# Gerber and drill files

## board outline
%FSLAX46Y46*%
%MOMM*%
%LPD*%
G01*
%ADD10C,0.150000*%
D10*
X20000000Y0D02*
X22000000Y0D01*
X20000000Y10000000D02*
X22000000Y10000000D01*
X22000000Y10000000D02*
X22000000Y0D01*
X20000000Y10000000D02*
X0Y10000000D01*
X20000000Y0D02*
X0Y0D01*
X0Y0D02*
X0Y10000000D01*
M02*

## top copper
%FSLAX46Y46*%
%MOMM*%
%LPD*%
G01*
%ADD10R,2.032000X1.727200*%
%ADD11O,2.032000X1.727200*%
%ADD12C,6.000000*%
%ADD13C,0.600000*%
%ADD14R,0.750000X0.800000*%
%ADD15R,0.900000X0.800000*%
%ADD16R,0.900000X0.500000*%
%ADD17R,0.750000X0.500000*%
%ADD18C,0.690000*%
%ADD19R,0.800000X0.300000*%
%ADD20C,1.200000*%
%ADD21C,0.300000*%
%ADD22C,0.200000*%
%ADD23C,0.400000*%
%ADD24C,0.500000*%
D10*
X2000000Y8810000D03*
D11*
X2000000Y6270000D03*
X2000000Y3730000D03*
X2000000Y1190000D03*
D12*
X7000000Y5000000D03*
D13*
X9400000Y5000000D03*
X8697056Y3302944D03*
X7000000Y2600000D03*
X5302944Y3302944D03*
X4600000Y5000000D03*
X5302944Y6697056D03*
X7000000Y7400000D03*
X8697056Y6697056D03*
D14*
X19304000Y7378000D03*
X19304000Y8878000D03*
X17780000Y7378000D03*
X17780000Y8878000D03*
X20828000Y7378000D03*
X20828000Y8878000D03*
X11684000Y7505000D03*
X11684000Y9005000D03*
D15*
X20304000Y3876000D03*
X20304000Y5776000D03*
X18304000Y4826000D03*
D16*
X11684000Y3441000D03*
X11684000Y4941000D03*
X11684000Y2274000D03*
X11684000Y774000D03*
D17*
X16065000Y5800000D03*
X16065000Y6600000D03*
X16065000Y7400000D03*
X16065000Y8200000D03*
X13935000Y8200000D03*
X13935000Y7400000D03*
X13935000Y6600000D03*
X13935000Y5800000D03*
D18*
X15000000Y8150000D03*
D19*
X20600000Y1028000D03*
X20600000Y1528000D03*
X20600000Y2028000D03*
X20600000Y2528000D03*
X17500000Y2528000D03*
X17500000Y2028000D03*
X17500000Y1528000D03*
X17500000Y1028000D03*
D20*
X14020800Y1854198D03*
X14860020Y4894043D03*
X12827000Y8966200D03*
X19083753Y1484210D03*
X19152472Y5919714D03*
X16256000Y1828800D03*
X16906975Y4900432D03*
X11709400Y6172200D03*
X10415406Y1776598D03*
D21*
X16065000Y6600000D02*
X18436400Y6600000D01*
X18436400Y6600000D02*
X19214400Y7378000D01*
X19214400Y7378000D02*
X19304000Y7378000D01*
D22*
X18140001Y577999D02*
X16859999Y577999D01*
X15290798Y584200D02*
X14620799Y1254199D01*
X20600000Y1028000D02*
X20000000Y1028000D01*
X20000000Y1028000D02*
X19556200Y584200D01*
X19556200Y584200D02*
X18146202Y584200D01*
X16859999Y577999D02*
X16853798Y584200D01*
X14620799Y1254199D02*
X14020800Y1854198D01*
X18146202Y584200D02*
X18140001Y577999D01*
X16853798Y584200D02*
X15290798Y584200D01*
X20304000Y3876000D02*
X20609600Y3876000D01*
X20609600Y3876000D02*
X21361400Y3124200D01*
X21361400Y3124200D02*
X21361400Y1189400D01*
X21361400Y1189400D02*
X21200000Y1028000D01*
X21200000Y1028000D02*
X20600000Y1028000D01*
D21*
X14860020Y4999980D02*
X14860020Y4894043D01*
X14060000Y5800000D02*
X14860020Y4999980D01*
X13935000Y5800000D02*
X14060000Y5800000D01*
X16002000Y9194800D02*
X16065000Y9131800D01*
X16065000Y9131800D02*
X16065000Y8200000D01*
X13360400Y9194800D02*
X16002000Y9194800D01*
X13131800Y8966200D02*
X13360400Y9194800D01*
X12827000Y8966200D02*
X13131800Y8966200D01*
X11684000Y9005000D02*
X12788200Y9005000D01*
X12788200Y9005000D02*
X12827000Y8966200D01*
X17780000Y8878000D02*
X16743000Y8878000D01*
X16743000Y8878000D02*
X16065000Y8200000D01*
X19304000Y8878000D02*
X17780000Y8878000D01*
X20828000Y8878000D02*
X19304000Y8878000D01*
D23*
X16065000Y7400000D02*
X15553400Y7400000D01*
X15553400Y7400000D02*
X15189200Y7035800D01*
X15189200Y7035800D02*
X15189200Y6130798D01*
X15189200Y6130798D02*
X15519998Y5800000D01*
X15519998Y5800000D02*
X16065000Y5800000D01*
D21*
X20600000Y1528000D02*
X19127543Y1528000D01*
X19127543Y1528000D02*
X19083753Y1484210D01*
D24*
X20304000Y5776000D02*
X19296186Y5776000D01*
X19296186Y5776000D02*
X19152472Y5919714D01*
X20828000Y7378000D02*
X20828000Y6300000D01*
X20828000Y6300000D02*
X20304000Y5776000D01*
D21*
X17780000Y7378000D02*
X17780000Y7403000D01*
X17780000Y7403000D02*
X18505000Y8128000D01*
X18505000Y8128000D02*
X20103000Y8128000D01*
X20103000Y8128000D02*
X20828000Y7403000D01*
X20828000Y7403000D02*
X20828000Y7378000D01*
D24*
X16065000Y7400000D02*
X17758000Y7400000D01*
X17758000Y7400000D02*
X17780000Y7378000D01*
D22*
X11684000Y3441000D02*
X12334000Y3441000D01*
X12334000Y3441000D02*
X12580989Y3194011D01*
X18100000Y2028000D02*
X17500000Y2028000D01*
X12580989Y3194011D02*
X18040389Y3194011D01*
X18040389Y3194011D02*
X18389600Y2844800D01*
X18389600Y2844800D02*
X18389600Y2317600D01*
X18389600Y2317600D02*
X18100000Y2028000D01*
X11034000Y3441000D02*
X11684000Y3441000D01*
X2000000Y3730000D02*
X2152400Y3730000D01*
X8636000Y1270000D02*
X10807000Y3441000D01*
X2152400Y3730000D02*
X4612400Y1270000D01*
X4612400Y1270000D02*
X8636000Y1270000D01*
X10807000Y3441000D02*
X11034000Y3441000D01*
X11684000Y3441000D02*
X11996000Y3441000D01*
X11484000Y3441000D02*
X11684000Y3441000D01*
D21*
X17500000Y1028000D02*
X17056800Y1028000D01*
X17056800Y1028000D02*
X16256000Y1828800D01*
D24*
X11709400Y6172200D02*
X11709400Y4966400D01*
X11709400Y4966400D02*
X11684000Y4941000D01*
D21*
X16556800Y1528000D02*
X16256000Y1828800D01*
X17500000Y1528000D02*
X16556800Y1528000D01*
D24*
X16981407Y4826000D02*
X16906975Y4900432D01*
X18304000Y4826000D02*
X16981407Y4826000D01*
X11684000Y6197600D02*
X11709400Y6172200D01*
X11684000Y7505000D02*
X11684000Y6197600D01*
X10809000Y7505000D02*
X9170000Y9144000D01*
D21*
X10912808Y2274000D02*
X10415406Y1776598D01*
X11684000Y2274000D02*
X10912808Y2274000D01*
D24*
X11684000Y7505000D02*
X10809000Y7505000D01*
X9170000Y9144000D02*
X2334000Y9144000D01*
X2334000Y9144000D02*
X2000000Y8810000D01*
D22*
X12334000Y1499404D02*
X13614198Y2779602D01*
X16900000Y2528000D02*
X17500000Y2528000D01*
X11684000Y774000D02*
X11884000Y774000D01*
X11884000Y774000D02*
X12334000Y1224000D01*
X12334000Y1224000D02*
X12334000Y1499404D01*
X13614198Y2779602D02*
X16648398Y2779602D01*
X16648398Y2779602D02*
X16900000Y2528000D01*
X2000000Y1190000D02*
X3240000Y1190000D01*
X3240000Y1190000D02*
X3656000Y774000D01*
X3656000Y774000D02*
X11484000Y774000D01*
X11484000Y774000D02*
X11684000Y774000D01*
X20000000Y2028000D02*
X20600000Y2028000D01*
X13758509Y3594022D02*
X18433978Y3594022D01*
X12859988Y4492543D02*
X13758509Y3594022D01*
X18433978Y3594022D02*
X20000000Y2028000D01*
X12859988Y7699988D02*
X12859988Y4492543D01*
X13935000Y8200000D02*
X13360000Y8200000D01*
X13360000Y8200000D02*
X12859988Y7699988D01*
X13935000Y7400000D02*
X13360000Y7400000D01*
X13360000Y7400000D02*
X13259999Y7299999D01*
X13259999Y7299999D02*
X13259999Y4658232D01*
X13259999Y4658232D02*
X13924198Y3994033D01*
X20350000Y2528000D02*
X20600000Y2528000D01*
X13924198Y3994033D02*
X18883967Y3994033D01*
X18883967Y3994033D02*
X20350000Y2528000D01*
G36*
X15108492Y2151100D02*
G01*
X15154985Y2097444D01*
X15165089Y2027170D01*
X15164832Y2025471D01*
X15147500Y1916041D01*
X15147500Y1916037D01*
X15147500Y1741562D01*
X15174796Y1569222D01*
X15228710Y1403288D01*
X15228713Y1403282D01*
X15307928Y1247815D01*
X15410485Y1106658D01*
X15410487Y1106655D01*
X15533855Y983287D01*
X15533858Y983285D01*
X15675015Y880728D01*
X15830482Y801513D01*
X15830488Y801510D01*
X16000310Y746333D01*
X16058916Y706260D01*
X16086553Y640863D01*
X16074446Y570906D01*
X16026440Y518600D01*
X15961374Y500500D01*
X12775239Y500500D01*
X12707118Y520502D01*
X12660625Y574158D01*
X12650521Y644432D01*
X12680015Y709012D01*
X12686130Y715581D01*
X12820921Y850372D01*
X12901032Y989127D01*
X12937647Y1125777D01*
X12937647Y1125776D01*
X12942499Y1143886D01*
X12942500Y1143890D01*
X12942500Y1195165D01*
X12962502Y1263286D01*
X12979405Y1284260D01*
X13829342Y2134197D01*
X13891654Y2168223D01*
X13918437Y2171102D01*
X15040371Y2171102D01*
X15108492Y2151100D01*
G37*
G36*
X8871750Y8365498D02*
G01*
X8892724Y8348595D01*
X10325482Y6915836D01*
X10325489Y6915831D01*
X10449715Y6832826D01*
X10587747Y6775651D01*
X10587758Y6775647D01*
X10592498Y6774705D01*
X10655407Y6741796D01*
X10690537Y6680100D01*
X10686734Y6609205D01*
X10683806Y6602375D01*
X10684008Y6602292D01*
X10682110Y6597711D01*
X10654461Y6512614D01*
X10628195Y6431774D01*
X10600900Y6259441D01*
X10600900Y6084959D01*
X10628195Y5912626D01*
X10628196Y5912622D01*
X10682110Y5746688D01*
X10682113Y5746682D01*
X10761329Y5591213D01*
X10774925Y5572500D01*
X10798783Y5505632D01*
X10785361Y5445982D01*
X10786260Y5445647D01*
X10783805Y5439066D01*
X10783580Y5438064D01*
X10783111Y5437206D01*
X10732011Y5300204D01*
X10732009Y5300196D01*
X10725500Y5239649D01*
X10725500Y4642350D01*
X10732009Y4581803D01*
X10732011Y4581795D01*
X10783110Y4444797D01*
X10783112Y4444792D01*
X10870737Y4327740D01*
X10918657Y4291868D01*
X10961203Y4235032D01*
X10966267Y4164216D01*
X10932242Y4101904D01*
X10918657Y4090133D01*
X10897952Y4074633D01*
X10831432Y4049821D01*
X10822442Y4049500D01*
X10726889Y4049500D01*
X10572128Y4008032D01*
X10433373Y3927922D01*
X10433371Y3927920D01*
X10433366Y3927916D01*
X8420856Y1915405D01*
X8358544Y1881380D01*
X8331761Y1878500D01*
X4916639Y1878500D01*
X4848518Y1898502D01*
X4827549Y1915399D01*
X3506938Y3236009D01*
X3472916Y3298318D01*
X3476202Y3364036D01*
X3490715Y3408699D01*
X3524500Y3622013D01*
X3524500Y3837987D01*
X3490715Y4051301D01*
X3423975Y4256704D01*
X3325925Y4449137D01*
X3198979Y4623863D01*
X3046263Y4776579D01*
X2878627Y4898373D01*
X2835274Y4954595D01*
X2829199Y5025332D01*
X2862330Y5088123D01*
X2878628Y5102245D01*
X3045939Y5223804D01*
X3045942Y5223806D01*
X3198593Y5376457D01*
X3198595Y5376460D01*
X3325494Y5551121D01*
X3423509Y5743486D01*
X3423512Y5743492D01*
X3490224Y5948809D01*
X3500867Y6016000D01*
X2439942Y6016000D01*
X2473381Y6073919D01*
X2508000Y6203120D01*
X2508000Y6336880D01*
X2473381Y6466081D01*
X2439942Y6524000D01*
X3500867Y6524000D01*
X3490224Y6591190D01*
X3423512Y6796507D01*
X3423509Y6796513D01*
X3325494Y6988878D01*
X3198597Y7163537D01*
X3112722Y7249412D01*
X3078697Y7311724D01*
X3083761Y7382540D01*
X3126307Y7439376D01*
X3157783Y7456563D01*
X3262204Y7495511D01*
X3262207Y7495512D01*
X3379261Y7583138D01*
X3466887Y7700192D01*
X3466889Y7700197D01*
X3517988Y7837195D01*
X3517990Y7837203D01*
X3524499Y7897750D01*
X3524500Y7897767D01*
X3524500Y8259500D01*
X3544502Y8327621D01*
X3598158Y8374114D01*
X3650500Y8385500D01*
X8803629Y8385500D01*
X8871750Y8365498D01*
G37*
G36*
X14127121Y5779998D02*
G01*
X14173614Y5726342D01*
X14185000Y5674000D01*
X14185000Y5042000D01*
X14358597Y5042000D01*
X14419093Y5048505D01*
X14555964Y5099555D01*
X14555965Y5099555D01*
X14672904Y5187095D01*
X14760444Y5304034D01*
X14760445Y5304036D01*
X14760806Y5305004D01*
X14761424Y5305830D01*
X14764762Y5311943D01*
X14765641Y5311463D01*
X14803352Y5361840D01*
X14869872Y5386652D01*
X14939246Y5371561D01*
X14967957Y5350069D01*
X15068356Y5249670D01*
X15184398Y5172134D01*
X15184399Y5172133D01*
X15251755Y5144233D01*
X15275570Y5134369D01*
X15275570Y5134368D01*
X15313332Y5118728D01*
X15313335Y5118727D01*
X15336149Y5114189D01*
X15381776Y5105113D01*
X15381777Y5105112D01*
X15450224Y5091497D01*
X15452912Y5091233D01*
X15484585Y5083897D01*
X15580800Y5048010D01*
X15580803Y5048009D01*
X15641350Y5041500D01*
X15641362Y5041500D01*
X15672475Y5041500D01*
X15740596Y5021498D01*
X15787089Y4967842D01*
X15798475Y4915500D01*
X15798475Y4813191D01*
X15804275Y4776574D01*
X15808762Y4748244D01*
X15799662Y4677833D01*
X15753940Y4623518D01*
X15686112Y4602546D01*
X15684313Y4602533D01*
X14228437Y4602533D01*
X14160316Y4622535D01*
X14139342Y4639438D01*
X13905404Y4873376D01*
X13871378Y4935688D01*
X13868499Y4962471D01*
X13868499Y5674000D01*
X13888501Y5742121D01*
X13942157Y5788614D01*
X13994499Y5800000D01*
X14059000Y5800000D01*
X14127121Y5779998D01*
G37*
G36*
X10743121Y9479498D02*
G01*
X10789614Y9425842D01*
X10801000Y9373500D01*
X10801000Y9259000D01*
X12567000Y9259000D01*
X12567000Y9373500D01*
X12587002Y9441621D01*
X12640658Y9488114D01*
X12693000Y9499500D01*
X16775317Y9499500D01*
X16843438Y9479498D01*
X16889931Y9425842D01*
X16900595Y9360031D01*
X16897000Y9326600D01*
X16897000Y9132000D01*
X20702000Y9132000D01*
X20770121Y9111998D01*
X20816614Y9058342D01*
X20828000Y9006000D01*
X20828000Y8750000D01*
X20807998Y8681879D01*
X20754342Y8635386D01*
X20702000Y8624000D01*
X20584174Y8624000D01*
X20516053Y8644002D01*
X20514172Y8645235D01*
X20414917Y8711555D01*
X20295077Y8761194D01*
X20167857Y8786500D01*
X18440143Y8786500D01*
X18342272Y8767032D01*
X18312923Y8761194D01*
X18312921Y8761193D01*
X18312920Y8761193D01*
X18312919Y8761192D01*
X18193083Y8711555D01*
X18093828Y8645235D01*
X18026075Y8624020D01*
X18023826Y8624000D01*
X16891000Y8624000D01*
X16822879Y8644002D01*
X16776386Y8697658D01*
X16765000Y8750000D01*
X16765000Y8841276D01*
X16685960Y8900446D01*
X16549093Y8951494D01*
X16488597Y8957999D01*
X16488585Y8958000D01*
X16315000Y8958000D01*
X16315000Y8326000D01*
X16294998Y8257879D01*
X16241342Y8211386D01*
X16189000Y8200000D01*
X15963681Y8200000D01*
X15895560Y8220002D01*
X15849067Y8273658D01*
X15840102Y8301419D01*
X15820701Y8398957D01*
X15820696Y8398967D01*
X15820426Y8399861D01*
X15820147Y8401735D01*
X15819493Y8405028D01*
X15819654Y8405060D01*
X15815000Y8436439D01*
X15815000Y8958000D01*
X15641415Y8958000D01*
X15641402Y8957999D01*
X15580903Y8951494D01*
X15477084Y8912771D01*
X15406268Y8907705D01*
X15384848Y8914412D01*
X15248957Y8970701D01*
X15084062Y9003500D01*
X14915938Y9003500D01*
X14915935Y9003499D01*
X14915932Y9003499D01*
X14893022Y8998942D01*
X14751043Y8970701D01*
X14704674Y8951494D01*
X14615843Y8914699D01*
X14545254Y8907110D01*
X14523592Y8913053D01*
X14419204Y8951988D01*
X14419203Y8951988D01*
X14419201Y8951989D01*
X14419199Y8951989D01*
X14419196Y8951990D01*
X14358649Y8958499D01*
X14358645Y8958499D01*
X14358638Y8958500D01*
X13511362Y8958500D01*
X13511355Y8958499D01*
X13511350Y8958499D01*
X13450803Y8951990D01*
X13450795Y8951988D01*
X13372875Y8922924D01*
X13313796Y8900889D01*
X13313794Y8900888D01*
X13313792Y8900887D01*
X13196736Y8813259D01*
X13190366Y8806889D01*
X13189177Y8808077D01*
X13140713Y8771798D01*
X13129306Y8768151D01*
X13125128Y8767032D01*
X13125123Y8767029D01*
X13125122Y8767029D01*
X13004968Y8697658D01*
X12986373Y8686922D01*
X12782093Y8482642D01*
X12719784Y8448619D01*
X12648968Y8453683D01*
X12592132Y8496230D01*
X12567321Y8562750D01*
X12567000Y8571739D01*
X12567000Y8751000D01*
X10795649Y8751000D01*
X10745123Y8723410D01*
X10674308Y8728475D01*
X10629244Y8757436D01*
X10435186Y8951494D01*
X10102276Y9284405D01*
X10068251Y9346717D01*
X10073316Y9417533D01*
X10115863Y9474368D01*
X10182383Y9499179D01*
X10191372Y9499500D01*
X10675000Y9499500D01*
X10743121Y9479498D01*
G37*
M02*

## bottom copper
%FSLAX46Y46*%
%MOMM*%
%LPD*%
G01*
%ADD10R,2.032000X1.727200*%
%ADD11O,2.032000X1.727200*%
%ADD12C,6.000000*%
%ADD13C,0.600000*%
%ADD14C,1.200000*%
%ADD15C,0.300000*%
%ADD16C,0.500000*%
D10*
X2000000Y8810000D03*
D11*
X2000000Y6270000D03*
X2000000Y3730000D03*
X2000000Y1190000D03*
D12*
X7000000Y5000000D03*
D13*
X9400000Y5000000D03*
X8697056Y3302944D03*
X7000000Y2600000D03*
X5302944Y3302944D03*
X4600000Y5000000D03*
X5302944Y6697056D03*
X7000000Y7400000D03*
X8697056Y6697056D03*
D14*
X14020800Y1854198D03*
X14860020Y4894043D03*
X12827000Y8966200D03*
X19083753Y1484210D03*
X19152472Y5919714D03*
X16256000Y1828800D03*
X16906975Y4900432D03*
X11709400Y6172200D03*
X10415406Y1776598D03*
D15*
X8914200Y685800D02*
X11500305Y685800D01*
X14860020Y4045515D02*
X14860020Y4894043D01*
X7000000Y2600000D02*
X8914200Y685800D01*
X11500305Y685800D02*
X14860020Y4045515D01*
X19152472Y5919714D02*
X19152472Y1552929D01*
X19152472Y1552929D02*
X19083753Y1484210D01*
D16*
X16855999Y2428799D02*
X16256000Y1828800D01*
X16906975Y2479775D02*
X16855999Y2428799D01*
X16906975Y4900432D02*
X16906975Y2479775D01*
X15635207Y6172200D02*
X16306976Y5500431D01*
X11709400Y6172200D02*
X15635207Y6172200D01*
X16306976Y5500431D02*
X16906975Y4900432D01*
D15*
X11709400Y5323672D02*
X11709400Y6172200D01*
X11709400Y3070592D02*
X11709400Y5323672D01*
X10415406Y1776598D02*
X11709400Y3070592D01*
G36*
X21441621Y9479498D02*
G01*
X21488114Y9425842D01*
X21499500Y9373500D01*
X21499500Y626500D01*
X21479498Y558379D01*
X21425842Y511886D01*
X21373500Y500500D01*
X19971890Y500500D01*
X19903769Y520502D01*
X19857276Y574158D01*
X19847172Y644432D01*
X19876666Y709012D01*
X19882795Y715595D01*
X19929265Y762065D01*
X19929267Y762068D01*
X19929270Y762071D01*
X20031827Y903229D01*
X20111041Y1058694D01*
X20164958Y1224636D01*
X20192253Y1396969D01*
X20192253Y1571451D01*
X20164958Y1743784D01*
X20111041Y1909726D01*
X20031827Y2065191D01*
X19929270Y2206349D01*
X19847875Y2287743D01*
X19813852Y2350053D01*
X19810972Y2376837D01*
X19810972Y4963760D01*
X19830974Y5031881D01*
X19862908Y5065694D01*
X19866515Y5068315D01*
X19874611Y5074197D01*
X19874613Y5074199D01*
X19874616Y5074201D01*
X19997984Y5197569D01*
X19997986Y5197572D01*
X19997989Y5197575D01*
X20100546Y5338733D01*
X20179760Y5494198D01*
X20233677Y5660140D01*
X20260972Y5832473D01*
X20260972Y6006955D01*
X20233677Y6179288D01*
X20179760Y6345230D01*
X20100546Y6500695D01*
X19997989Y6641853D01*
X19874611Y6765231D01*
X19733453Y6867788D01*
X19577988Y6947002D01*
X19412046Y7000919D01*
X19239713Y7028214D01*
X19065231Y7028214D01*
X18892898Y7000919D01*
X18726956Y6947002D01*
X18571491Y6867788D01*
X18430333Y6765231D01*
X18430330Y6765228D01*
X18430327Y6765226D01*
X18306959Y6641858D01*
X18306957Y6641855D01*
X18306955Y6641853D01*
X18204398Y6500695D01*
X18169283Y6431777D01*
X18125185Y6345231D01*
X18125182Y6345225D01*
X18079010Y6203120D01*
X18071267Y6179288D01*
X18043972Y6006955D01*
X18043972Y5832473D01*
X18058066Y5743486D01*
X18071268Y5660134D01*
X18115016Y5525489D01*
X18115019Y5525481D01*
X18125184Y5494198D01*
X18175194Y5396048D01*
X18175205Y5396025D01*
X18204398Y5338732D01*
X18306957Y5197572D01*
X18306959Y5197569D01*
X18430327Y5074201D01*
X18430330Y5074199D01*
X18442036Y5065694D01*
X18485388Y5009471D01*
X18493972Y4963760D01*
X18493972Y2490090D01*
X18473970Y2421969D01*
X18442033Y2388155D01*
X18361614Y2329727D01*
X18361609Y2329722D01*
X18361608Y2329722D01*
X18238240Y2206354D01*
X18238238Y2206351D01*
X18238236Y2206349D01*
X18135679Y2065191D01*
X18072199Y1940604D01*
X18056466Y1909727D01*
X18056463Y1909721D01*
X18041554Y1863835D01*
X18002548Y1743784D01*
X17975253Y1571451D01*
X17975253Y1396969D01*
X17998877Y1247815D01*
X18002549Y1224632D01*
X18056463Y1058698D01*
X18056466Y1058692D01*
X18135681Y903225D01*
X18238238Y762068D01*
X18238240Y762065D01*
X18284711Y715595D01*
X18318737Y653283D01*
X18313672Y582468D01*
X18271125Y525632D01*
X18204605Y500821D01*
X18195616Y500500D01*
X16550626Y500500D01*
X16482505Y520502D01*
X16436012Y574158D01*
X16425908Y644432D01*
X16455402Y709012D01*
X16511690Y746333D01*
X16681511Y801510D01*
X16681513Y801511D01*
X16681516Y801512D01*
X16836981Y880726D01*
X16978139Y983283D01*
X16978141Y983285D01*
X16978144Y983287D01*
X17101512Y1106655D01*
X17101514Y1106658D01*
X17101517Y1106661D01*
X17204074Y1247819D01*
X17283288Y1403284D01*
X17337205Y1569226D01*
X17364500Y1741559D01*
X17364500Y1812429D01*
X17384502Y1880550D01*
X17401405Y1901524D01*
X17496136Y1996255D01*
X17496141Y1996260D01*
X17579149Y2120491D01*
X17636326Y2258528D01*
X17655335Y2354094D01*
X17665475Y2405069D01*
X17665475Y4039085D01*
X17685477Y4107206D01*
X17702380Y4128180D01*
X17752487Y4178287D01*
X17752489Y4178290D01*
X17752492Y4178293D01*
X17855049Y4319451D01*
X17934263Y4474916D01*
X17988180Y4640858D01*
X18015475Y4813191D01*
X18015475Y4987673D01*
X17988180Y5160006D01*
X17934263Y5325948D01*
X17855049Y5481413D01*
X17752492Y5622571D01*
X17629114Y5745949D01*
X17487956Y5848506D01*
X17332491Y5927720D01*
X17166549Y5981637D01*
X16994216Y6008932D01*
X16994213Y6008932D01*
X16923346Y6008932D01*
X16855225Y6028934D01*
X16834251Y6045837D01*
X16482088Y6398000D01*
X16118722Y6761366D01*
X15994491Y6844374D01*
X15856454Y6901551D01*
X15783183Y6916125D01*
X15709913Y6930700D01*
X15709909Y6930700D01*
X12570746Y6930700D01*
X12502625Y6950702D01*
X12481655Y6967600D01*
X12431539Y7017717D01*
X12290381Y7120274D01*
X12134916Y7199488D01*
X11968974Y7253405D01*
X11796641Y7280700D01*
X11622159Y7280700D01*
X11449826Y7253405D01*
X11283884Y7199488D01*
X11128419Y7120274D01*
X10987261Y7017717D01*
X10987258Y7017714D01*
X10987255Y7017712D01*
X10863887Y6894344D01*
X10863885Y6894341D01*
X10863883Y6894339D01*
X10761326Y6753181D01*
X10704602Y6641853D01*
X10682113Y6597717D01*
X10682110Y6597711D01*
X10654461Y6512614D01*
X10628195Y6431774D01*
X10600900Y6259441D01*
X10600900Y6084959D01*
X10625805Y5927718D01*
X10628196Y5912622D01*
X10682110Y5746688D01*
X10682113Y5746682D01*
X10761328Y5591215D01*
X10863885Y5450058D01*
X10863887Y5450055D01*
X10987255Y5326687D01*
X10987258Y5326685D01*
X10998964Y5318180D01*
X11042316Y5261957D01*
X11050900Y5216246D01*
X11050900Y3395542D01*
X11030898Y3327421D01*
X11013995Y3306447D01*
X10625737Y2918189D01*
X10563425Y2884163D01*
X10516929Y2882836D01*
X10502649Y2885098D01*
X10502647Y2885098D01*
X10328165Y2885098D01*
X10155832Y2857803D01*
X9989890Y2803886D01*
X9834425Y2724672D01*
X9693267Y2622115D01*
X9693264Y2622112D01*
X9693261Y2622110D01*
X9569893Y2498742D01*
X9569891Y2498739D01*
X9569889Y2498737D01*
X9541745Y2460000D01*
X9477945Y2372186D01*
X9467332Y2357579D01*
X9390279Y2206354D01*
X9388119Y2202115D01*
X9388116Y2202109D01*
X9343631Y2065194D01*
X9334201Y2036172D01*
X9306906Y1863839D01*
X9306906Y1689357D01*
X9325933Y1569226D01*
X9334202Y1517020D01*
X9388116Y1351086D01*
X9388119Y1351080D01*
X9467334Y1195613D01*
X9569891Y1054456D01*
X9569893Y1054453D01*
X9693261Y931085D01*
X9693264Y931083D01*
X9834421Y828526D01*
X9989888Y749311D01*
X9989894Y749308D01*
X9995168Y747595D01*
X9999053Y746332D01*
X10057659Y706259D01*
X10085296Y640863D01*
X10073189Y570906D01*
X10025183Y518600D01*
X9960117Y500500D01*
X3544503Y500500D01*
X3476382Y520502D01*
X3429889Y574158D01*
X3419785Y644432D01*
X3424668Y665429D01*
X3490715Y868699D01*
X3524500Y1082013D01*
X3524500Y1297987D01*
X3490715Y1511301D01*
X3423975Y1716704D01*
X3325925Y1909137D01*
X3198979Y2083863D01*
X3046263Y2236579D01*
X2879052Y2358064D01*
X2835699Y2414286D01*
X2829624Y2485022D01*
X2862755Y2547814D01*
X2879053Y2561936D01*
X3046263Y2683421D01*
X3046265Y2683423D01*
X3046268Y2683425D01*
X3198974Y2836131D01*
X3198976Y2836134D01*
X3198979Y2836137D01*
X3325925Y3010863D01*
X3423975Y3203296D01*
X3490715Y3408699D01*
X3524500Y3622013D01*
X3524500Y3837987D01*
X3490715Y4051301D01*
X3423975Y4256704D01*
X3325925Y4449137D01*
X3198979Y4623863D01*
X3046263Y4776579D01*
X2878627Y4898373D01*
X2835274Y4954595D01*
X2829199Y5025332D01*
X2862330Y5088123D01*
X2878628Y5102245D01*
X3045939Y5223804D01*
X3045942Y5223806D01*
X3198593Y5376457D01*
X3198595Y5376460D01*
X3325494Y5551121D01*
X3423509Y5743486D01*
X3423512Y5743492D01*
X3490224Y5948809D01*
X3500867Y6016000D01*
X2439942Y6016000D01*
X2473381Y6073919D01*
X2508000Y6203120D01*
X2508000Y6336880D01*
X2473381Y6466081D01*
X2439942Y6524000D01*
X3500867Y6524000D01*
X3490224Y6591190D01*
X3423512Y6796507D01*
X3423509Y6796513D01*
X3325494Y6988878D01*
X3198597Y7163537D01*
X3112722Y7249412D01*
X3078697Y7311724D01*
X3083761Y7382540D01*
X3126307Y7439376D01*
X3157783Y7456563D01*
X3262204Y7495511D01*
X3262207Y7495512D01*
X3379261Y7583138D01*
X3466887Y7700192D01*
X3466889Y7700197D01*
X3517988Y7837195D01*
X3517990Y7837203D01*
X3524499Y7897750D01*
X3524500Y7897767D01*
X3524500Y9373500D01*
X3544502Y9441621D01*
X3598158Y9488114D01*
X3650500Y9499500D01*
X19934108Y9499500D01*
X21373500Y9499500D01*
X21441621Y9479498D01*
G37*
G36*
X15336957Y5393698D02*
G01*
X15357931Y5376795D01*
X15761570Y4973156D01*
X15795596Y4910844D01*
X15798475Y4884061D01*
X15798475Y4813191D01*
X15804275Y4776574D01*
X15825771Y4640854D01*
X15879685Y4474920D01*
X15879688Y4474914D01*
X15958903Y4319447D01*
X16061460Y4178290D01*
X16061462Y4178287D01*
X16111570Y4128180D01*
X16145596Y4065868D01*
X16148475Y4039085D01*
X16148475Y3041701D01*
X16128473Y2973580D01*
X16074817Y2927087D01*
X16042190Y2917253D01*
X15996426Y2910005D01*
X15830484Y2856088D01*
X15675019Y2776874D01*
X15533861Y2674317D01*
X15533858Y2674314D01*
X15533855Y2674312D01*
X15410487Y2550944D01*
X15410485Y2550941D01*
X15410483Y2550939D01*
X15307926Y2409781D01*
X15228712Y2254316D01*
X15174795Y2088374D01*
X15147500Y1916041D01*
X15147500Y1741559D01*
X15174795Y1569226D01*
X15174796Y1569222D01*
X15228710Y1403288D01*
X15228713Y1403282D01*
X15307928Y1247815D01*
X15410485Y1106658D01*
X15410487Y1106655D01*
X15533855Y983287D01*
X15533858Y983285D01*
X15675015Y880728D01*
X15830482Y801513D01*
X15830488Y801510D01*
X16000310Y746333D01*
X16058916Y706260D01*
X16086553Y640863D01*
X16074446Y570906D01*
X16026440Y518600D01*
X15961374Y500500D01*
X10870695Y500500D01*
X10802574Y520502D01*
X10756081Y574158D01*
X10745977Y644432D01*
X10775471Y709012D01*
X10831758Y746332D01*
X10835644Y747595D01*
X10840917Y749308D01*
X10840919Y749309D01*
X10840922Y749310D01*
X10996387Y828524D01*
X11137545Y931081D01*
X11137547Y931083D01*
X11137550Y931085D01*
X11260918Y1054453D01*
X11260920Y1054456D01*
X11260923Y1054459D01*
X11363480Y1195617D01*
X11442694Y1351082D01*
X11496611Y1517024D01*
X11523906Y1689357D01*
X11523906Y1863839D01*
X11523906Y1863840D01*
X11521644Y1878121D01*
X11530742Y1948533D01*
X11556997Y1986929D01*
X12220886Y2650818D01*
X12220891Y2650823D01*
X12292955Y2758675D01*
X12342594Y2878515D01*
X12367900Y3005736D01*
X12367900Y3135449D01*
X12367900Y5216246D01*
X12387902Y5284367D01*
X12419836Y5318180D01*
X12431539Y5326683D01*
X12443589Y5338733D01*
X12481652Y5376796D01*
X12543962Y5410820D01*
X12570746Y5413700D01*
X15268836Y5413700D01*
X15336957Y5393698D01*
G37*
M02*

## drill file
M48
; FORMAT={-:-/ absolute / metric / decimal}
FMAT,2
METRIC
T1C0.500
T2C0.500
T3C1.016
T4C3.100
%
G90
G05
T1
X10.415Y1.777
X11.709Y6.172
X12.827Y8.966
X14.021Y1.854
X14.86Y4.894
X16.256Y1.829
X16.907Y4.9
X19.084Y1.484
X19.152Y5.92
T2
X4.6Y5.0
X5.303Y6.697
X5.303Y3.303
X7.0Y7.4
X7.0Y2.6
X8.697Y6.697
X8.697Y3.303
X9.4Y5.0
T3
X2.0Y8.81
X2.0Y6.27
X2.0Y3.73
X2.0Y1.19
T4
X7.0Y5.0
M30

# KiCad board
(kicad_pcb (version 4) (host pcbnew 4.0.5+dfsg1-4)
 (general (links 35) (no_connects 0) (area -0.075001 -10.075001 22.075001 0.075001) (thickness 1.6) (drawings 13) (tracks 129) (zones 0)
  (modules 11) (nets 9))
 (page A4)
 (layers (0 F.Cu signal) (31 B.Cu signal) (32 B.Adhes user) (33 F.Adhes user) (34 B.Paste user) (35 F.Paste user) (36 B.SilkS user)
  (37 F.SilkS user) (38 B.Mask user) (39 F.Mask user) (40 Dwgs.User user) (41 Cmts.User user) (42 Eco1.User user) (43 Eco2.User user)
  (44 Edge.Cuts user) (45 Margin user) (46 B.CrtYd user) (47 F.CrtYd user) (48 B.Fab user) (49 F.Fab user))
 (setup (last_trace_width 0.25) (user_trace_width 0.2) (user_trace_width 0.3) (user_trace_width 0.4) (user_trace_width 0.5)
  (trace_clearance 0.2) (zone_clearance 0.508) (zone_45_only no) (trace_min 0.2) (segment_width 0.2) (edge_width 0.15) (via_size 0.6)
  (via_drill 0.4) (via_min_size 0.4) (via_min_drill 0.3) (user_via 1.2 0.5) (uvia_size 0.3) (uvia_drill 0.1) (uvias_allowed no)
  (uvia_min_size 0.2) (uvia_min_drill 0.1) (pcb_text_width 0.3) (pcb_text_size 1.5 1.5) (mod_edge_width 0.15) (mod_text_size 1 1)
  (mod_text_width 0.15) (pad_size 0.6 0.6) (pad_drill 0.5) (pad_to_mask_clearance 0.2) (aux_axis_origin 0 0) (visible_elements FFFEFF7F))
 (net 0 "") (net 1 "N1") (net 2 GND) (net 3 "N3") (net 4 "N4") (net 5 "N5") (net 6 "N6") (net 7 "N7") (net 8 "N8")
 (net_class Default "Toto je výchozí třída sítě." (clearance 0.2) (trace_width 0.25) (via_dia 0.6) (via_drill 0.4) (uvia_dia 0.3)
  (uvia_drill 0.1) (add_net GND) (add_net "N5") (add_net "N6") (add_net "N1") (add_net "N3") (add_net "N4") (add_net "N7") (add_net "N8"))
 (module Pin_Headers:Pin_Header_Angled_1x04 (layer B.Cu) (at 2 -8.81 180)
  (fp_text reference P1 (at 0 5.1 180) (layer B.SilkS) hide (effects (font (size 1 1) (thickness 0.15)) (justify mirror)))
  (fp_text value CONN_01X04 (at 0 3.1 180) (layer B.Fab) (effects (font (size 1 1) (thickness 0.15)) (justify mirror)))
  (pad 1 thru_hole rect (at 0 0 180) (size 2.032 1.7272) (drill 1.016) (layers *.Cu *.Mask) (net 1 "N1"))
  (pad 2 thru_hole oval (at 0 -2.54 180) (size 2.032 1.7272) (drill 1.016) (layers *.Cu *.Mask) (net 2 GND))
  (pad 3 thru_hole oval (at 0 -5.08 180) (size 2.032 1.7272) (drill 1.016) (layers *.Cu *.Mask) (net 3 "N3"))
  (pad 4 thru_hole oval (at 0 -7.62 180) (size 2.032 1.7272) (drill 1.016) (layers *.Cu *.Mask) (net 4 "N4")))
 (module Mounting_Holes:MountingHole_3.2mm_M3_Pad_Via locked (layer F.Cu) (at 7 -5)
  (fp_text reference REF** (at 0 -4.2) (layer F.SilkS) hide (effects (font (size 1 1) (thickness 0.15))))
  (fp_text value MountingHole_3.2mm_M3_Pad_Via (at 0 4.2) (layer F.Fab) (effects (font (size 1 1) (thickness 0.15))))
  (pad 1 thru_hole circle (at 0 0) (size 6 6) (drill 3.1) (layers *.Cu *.Mask) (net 2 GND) (zone_connect 2))
  (pad "" thru_hole circle (at 2.4 0) (size 0.6 0.6) (drill 0.5) (layers *.Cu *.Mask) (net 2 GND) (zone_connect 2))
  (pad "" thru_hole circle (at 1.697056 1.697056) (size 0.6 0.6) (drill 0.5) (layers *.Cu *.Mask) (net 2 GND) (zone_connect 2))
  (pad "" thru_hole circle (at 0 2.4) (size 0.6 0.6) (drill 0.5) (layers *.Cu *.Mask) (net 2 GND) (zone_connect 2))
  (pad "" thru_hole circle (at -1.697056 1.697056) (size 0.6 0.6) (drill 0.5) (layers *.Cu *.Mask) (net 2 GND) (zone_connect 2))
  (pad "" thru_hole circle (at -2.4 0) (size 0.6 0.6) (drill 0.5) (layers *.Cu *.Mask) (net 2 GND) (zone_connect 2))
  (pad "" thru_hole circle (at -1.697056 -1.697056) (size 0.6 0.6) (drill 0.5) (layers *.Cu *.Mask) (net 2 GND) (zone_connect 2))
  (pad "" thru_hole circle (at 0 -2.4) (size 0.6 0.6) (drill 0.5) (layers *.Cu *.Mask) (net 2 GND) (zone_connect 2))
  (pad "" thru_hole circle (at 1.697056 -1.697056) (size 0.6 0.6) (drill 0.5) (layers *.Cu *.Mask) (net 2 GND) (zone_connect 2)))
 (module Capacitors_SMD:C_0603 (layer F.Cu) (at 19.304 -8.128 90)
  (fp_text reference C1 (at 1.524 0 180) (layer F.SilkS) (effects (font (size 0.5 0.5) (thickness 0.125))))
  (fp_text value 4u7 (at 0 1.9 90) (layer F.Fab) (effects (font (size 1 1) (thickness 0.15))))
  (pad 1 smd rect (at -0.75 0 90) (size 0.8 0.75) (layers F.Cu F.Paste F.Mask) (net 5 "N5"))
  (pad 2 smd rect (at 0.75 0 90) (size 0.8 0.75) (layers F.Cu F.Paste F.Mask) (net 2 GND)))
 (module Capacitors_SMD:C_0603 (layer F.Cu) (at 17.78 -8.128 90)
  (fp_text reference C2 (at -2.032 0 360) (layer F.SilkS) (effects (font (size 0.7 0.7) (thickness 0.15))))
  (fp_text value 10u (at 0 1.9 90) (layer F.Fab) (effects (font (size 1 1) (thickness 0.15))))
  (pad 1 smd rect (at -0.75 0 90) (size 0.8 0.75) (layers F.Cu F.Paste F.Mask) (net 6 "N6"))
  (pad 2 smd rect (at 0.75 0 90) (size 0.8 0.75) (layers F.Cu F.Paste F.Mask) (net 2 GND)))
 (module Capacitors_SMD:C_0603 (layer F.Cu) (at 20.828 -8.128 90)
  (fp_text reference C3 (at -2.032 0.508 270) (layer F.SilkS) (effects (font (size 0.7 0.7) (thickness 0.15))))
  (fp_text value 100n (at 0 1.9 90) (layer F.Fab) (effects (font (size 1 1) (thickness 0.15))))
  (pad 1 smd rect (at -0.75 0 90) (size 0.8 0.75) (layers F.Cu F.Paste F.Mask) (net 6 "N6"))
  (pad 2 smd rect (at 0.75 0 90) (size 0.8 0.75) (layers F.Cu F.Paste F.Mask) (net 2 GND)))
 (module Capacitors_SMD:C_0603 (layer F.Cu) (at 11.684 -8.255 90)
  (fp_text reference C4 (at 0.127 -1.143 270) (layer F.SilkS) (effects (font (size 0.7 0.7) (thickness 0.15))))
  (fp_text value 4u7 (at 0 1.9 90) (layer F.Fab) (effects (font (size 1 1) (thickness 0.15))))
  (pad 1 smd rect (at -0.75 0 90) (size 0.8 0.75) (layers F.Cu F.Paste F.Mask) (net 1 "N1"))
  (pad 2 smd rect (at 0.75 0 90) (size 0.8 0.75) (layers F.Cu F.Paste F.Mask) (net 2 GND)))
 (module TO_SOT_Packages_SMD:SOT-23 (layer F.Cu) (at 19.304 -4.826 180)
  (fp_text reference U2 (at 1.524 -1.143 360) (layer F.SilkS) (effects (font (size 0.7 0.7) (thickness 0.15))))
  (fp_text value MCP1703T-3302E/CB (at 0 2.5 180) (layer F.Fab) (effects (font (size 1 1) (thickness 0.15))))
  (pad 1 smd rect (at -1 -0.95 180) (size 0.9 0.8) (layers F.Cu F.Paste F.Mask) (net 2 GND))
  (pad 2 smd rect (at -1 0.95 180) (size 0.9 0.8) (layers F.Cu F.Paste F.Mask) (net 6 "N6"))
  (pad 3 smd rect (at 1 0 180) (size 0.9 0.8) (layers F.Cu F.Paste F.Mask) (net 1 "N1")))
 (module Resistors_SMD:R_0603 (layer F.Cu) (at 11.684 -4.191 90)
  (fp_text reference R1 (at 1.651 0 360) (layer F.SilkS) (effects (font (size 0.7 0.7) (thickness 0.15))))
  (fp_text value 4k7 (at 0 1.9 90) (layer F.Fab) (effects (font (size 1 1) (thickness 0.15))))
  (pad 1 smd rect (at -0.75 0 90) (size 0.5 0.9) (layers F.Cu F.Paste F.Mask) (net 3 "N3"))
  (pad 2 smd rect (at 0.75 0 90) (size 0.5 0.9) (layers F.Cu F.Paste F.Mask) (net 1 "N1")))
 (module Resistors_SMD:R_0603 (layer F.Cu) (at 11.684 -1.524 270)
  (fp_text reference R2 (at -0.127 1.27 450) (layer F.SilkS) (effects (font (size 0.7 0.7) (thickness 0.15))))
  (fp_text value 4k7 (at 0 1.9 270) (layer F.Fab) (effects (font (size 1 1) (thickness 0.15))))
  (pad 1 smd rect (at -0.75 0 270) (size 0.5 0.9) (layers F.Cu F.Paste F.Mask) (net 1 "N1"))
  (pad 2 smd rect (at 0.75 0 270) (size 0.5 0.9) (layers F.Cu F.Paste F.Mask) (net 4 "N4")))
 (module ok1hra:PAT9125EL (layer F.Cu) (at 15 -7 90)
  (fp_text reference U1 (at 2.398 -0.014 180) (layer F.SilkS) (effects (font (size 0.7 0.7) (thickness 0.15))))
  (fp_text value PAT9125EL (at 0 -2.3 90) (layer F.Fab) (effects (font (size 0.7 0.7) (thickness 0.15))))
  (pad 1 smd rect (at -1.2 1.065 90) (size 0.5 0.75) (layers F.Cu F.Paste F.Mask) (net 6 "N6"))
  (pad 2 smd rect (at -0.4 1.065 90) (size 0.5 0.75) (layers F.Cu F.Paste F.Mask) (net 5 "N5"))
  (pad 3 smd rect (at 0.4 1.065 90) (size 0.5 0.75) (layers F.Cu F.Paste F.Mask) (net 6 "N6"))
  (pad 4 smd rect (at 1.2 1.065 90) (size 0.5 0.75) (layers F.Cu F.Paste F.Mask) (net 2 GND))
  (pad 5 smd rect (at 1.2 -1.065 90) (size 0.5 0.75) (layers F.Cu F.Paste F.Mask) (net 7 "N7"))
  (pad 6 smd rect (at 0.4 -1.065 90) (size 0.5 0.75) (layers F.Cu F.Paste F.Mask) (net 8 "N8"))
  (pad 7 smd rect (at -0.4 -1.065 90) (size 0.5 0.75) (layers F.Cu F.Paste F.Mask))
  (pad 8 smd rect (at -1.2 -1.065 90) (size 0.5 0.75) (layers F.Cu F.Paste F.Mask) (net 2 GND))
  (pad 9 smd circle (at 1.15 0 90) (size 0.69 0.69) (layers F.Cu F.Paste F.Mask)))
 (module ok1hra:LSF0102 (layer F.Cu) (at 19.05 -1.778 270)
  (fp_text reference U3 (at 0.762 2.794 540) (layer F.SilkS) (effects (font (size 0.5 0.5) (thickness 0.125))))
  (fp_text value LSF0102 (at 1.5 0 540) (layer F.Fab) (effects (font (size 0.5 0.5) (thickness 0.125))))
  (pad 1 smd rect (at 0.75 -1.55 90) (size 0.3 0.8) (layers F.Cu F.Paste F.Mask) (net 2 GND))
  (pad 2 smd rect (at 0.25 -1.55 90) (size 0.3 0.8) (layers F.Cu F.Paste F.Mask) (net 6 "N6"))
  (pad 3 smd rect (at -0.25 -1.55 90) (size 0.3 0.8) (layers F.Cu F.Paste F.Mask) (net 7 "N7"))
  (pad 4 smd rect (at -0.75 -1.55 90) (size 0.3 0.8) (layers F.Cu F.Paste F.Mask) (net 8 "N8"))
  (pad 5 smd rect (at -0.75 1.55 90) (size 0.3 0.8) (layers F.Cu F.Paste F.Mask) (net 4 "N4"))
  (pad 6 smd rect (at -0.25 1.55 90) (size 0.3 0.8) (layers F.Cu F.Paste F.Mask) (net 3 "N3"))
  (pad 7 smd rect (at 0.25 1.55 90) (size 0.3 0.8) (layers F.Cu F.Paste F.Mask) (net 1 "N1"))
  (pad 8 smd rect (at 0.75 1.55 90) (size 0.3 0.8) (layers F.Cu F.Paste F.Mask) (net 1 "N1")))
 (gr_line (start 20 0) (end 22 0) (layer Edge.Cuts) (width 0.15))
 (gr_line (start 20 -10) (end 22 -10) (layer Edge.Cuts) (width 0.15))
 (gr_line (start 22 -10) (end 22 0) (layer Edge.Cuts) (width 0.15))
 (gr_line (start 20 -10) (end 0 -10) (layer Edge.Cuts) (width 0.15))
 (gr_line (start 20 0) (end 0 0) (angle 90) (layer Edge.Cuts) (width 0.15))
 (gr_line (start 0 0) (end 0 -10) (angle 90) (layer Edge.Cuts) (width 0.15))
 (segment (start 16.065 -6.6) (end 18.4364 -6.6) (width 0.3) (layer F.Cu) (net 5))
 (segment (start 18.4364 -6.6) (end 19.2144 -7.378) (width 0.3) (layer F.Cu) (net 5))
 (segment (start 19.2144 -7.378) (end 19.304 -7.378) (width 0.3) (layer F.Cu) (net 5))
 (segment (start 18.140001 -0.577999) (end 16.859999 -0.577999) (width 0.2) (layer F.Cu) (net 2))
 (segment (start 15.290798 -0.5842) (end 14.620799 -1.254199) (width 0.2) (layer F.Cu) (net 2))
 (segment (start 20.6 -1.028) (end 20 -1.028) (width 0.2) (layer F.Cu) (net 2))
 (segment (start 20 -1.028) (end 19.5562 -0.5842) (width 0.2) (layer F.Cu) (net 2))
 (segment (start 19.5562 -0.5842) (end 18.146202 -0.5842) (width 0.2) (layer F.Cu) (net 2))
 (segment (start 16.859999 -0.577999) (end 16.853798 -0.5842) (width 0.2) (layer F.Cu) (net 2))
 (segment (start 14.620799 -1.254199) (end 14.0208 -1.854198) (width 0.2) (layer F.Cu) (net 2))
 (segment (start 18.146202 -0.5842) (end 18.140001 -0.577999) (width 0.2) (layer F.Cu) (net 2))
 (segment (start 16.853798 -0.5842) (end 15.290798 -0.5842) (width 0.2) (layer F.Cu) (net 2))
 (via (at 14.0208 -1.854198) (size 1.2) (drill 0.5) (layers F.Cu B.Cu) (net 2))
 (segment (start 20.304 -3.876) (end 20.6096 -3.876) (width 0.2) (layer F.Cu) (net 2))
 (segment (start 20.6096 -3.876) (end 21.3614 -3.1242) (width 0.2) (layer F.Cu) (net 2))
 (segment (start 21.3614 -3.1242) (end 21.3614 -1.1894) (width 0.2) (layer F.Cu) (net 2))
 (segment (start 21.3614 -1.1894) (end 21.2 -1.028) (width 0.2) (layer F.Cu) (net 2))
 (segment (start 21.2 -1.028) (end 20.6 -1.028) (width 0.2) (layer F.Cu) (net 2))
 (segment (start 14.86002 -4.99998) (end 14.86002 -4.894043) (width 0.3) (layer F.Cu) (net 2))
 (segment (start 14.06 -5.8) (end 14.86002 -4.99998) (width 0.3) (layer F.Cu) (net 2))
 (segment (start 13.935 -5.8) (end 14.06 -5.8) (width 0.3) (layer F.Cu) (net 2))
 (segment (start 8.9142 -0.6858) (end 11.500305 -0.6858) (width 0.3) (layer B.Cu) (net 2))
 (segment (start 14.86002 -4.045515) (end 14.86002 -4.894043) (width 0.3) (layer B.Cu) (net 2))
 (segment (start 7 -2.6) (end 8.9142 -0.6858) (width 0.3) (layer B.Cu) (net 2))
 (via (at 14.86002 -4.894043) (size 1.2) (drill 0.5) (layers F.Cu B.Cu) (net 2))
 (segment (start 11.500305 -0.6858) (end 14.86002 -4.045515) (width 0.3) (layer B.Cu) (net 2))
 (segment (start 16.002 -9.1948) (end 16.065 -9.1318) (width 0.3) (layer F.Cu) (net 2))
 (segment (start 16.065 -9.1318) (end 16.065 -8.2) (width 0.3) (layer F.Cu) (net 2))
 (segment (start 13.3604 -9.1948) (end 16.002 -9.1948) (width 0.3) (layer F.Cu) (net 2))
 (segment (start 13.1318 -8.9662) (end 13.3604 -9.1948) (width 0.3) (layer F.Cu) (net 2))
 (segment (start 12.827 -8.9662) (end 13.1318 -8.9662) (width 0.3) (layer F.Cu) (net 2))
 (segment (start 11.684 -9.005) (end 12.7882 -9.005) (width 0.3) (layer F.Cu) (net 2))
 (segment (start 12.7882 -9.005) (end 12.827 -8.9662) (width 0.3) (layer F.Cu) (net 2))
 (via (at 12.827 -8.9662) (size 1.2) (drill 0.5) (layers F.Cu B.Cu) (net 2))
 (segment (start 17.78 -8.878) (end 16.743 -8.878) (width 0.3) (layer F.Cu) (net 2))
 (segment (start 16.743 -8.878) (end 16.065 -8.2) (width 0.3) (layer F.Cu) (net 2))
 (segment (start 19.304 -8.878) (end 17.78 -8.878) (width 0.3) (layer F.Cu) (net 2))
 (segment (start 20.828 -8.878) (end 19.304 -8.878) (width 0.3) (layer F.Cu) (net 2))
 (segment (start 16.065 -7.4) (end 15.5534 -7.4) (width 0.4) (layer F.Cu) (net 6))
 (segment (start 15.5534 -7.4) (end 15.1892 -7.0358) (width 0.4) (layer F.Cu) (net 6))
 (segment (start 15.1892 -7.0358) (end 15.1892 -6.130798) (width 0.4) (layer F.Cu) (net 6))
 (segment (start 15.1892 -6.130798) (end 15.519998 -5.8) (width 0.4) (layer F.Cu) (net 6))
 (segment (start 15.519998 -5.8) (end 16.065 -5.8) (width 0.4) (layer F.Cu) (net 6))
 (segment (start 20.6 -1.528) (end 19.127543 -1.528) (width 0.3) (layer F.Cu) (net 6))
 (segment (start 19.152472 -5.919714) (end 19.152472 -1.552929) (width 0.3) (layer B.Cu) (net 6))
 (segment (start 19.152472 -1.552929) (end 19.083753 -1.48421) (width 0.3) (layer B.Cu) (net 6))
 (via (at 19.083753 -1.48421) (size 1.2) (drill 0.5) (layers F.Cu B.Cu) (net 6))
 (segment (start 19.127543 -1.528) (end 19.083753 -1.48421) (width 0.3) (layer F.Cu) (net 6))
 (segment (start 20.304 -5.776) (end 19.296186 -5.776) (width 0.5) (layer F.Cu) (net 6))
 (segment (start 19.296186 -5.776) (end 19.152472 -5.919714) (width 0.5) (layer F.Cu) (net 6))
 (via (at 19.152472 -5.919714) (size 1.2) (drill 0.5) (layers F.Cu B.Cu) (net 6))
 (segment (start 20.828 -7.378) (end 20.828 -6.3) (width 0.5) (layer F.Cu) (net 6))
 (segment (start 20.828 -6.3) (end 20.304 -5.776) (width 0.5) (layer F.Cu) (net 6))
 (segment (start 17.78 -7.378) (end 17.78 -7.403) (width 0.3) (layer F.Cu) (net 6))
 (segment (start 17.78 -7.403) (end 18.505 -8.128) (width 0.3) (layer F.Cu) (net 6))
 (segment (start 18.505 -8.128) (end 20.103 -8.128) (width 0.3) (layer F.Cu) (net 6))
 (segment (start 20.103 -8.128) (end 20.828 -7.403) (width 0.3) (layer F.Cu) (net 6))
 (segment (start 20.828 -7.403) (end 20.828 -7.378) (width 0.3) (layer F.Cu) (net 6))
 (segment (start 16.065 -7.4) (end 17.758 -7.4) (width 0.5) (layer F.Cu) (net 6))
 (segment (start 17.758 -7.4) (end 17.78 -7.378) (width 0.5) (layer F.Cu) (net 6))
 (segment (start 11.684 -3.441) (end 12.334 -3.441) (width 0.2) (layer F.Cu) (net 3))
 (segment (start 12.334 -3.441) (end 12.580989 -3.194011) (width 0.2) (layer F.Cu) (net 3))
 (segment (start 18.1 -2.028) (end 17.5 -2.028) (width 0.2) (layer F.Cu) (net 3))
 (segment (start 12.580989 -3.194011) (end 18.040389 -3.194011) (width 0.2) (layer F.Cu) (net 3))
 (segment (start 18.040389 -3.194011) (end 18.3896 -2.8448) (width 0.2) (layer F.Cu) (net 3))
 (segment (start 18.3896 -2.8448) (end 18.3896 -2.3176) (width 0.2) (layer F.Cu) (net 3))
 (segment (start 18.3896 -2.3176) (end 18.1 -2.028) (width 0.2) (layer F.Cu) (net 3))
 (segment (start 11.034 -3.441) (end 11.684 -3.441) (width 0.2) (layer F.Cu) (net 3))
 (segment (start 2 -3.73) (end 2.1524 -3.73) (width 0.2) (layer F.Cu) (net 3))
 (segment (start 8.636 -1.27) (end 10.807 -3.441) (width 0.2) (layer F.Cu) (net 3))
 (segment (start 2.1524 -3.73) (end 4.6124 -1.27) (width 0.2) (layer F.Cu) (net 3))
 (segment (start 4.6124 -1.27) (end 8.636 -1.27) (width 0.2) (layer F.Cu) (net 3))
 (segment (start 10.807 -3.441) (end 11.034 -3.441) (width 0.2) (layer F.Cu) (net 3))
 (segment (start 11.684 -3.441) (end 11.996 -3.441) (width 0.2) (layer F.Cu) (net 3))
 (segment (start 11.484 -3.441) (end 11.684 -3.441) (width 0.2) (layer F.Cu) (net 3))
 (segment (start 17.5 -1.028) (end 17.0568 -1.028) (width 0.3) (layer F.Cu) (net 1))
 (segment (start 17.0568 -1.028) (end 16.256 -1.8288) (width 0.3) (layer F.Cu) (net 1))
 (segment (start 11.7094 -6.1722) (end 11.7094 -4.9664) (width 0.5) (layer F.Cu) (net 1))
 (segment (start 11.7094 -4.9664) (end 11.684 -4.941) (width 0.5) (layer F.Cu) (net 1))
 (segment (start 16.855999 -2.428799) (end 16.256 -1.8288) (width 0.5) (layer B.Cu) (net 1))
 (segment (start 16.906975 -2.479775) (end 16.855999 -2.428799) (width 0.5) (layer B.Cu) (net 1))
 (segment (start 16.906975 -4.900432) (end 16.906975 -2.479775) (width 0.5) (layer B.Cu) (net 1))
 (segment (start 16.5568 -1.528) (end 16.256 -1.8288) (width 0.3) (layer F.Cu) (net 1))
 (via (at 16.256 -1.8288) (size 1.2) (drill 0.5) (layers F.Cu B.Cu) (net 1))
 (segment (start 17.5 -1.528) (end 16.5568 -1.528) (width 0.3) (layer F.Cu) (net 1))
 (segment (start 16.981407 -4.826) (end 16.906975 -4.900432) (width 0.5) (layer F.Cu) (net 1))
 (segment (start 15.635207 -6.1722) (end 16.306976 -5.500431) (width 0.5) (layer B.Cu) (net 1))
 (segment (start 18.304 -4.826) (end 16.981407 -4.826) (width 0.5) (layer F.Cu) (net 1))
 (via (at 16.906975 -4.900432) (size 1.2) (drill 0.5) (layers F.Cu B.Cu) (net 1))
 (segment (start 11.7094 -6.1722) (end 15.635207 -6.1722) (width 0.5) (layer B.Cu) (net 1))
 (segment (start 16.306976 -5.500431) (end 16.906975 -4.900432) (width 0.5) (layer B.Cu) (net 1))
 (segment (start 11.7094 -5.323672) (end 11.7094 -6.1722) (width 0.3) (layer B.Cu) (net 1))
 (segment (start 11.7094 -3.070592) (end 11.7094 -5.323672) (width 0.3) (layer B.Cu) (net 1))
 (segment (start 10.415406 -1.776598) (end 11.7094 -3.070592) (width 0.3) (layer B.Cu) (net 1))
 (segment (start 11.684 -6.1976) (end 11.7094 -6.1722) (width 0.5) (layer F.Cu) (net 1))
 (segment (start 11.684 -7.505) (end 11.684 -6.1976) (width 0.5) (layer F.Cu) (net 1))
 (via (at 11.7094 -6.1722) (size 1.2) (drill 0.5) (layers F.Cu B.Cu) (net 1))
 (segment (start 10.809 -7.505) (end 9.17 -9.144) (width 0.5) (layer F.Cu) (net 1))
 (segment (start 10.912808 -2.274) (end 10.415406 -1.776598) (width 0.3) (layer F.Cu) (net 1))
 (via (at 10.415406 -1.776598) (size 1.2) (drill 0.5) (layers F.Cu B.Cu) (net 1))
 (segment (start 11.684 -2.274) (end 10.912808 -2.274) (width 0.3) (layer F.Cu) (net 1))
 (segment (start 11.684 -7.505) (end 10.809 -7.505) (width 0.5) (layer F.Cu) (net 1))
 (segment (start 9.17 -9.144) (end 2.334 -9.144) (width 0.5) (layer F.Cu) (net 1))
 (segment (start 2.334 -9.144) (end 2 -8.81) (width 0.5) (layer F.Cu) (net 1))
 (segment (start 12.334 -1.499404) (end 13.614198 -2.779602) (width 0.2) (layer F.Cu) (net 4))
 (segment (start 16.9 -2.528) (end 17.5 -2.528) (width 0.2) (layer F.Cu) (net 4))
 (segment (start 11.684 -0.774) (end 11.884 -0.774) (width 0.2) (layer F.Cu) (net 4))
 (segment (start 11.884 -0.774) (end 12.334 -1.224) (width 0.2) (layer F.Cu) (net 4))
 (segment (start 12.334 -1.224) (end 12.334 -1.499404) (width 0.2) (layer F.Cu) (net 4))
 (segment (start 13.614198 -2.779602) (end 16.648398 -2.779602) (width 0.2) (layer F.Cu) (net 4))
 (segment (start 16.648398 -2.779602) (end 16.9 -2.528) (width 0.2) (layer F.Cu) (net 4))
 (segment (start 2 -1.19) (end 3.24 -1.19) (width 0.2) (layer F.Cu) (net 4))
 (segment (start 3.24 -1.19) (end 3.656 -0.774) (width 0.2) (layer F.Cu) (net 4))
 (segment (start 3.656 -0.774) (end 11.484 -0.774) (width 0.2) (layer F.Cu) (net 4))
 (segment (start 11.484 -0.774) (end 11.684 -0.774) (width 0.2) (layer F.Cu) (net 4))
 (segment (start 20 -2.028) (end 20.6 -2.028) (width 0.2) (layer F.Cu) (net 7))
 (segment (start 13.758509 -3.594022) (end 18.433978 -3.594022) (width 0.2) (layer F.Cu) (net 7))
 (segment (start 12.859988 -4.492543) (end 13.758509 -3.594022) (width 0.2) (layer F.Cu) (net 7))
 (segment (start 18.433978 -3.594022) (end 20 -2.028) (width 0.2) (layer F.Cu) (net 7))
 (segment (start 12.859988 -7.699988) (end 12.859988 -4.492543) (width 0.2) (layer F.Cu) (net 7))
 (segment (start 13.935 -8.2) (end 13.36 -8.2) (width 0.2) (layer F.Cu) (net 7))
 (segment (start 13.36 -8.2) (end 12.859988 -7.699988) (width 0.2) (layer F.Cu) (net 7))
 (segment (start 13.935 -7.4) (end 13.36 -7.4) (width 0.2) (layer F.Cu) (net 8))
 (segment (start 13.36 -7.4) (end 13.259999 -7.299999) (width 0.2) (layer F.Cu) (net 8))
 (segment (start 13.259999 -7.299999) (end 13.259999 -4.658232) (width 0.2) (layer F.Cu) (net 8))
 (segment (start 13.259999 -4.658232) (end 13.924198 -3.994033) (width 0.2) (layer F.Cu) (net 8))
 (segment (start 20.35 -2.528) (end 20.6 -2.528) (width 0.2) (layer F.Cu) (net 8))
 (segment (start 13.924198 -3.994033) (end 18.883967 -3.994033) (width 0.2) (layer F.Cu) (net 8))
 (segment (start 18.883967 -3.994033) (end 20.35 -2.528) (width 0.2) (layer F.Cu) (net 8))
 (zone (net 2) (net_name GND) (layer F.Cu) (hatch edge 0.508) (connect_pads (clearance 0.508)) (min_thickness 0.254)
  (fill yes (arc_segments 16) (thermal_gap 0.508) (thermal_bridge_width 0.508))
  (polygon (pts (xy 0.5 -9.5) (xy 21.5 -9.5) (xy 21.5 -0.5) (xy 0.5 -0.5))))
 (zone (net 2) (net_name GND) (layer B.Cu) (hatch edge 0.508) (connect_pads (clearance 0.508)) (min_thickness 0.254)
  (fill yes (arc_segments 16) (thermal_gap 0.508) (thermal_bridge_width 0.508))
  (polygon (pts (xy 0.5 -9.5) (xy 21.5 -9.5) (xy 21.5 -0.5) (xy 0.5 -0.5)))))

